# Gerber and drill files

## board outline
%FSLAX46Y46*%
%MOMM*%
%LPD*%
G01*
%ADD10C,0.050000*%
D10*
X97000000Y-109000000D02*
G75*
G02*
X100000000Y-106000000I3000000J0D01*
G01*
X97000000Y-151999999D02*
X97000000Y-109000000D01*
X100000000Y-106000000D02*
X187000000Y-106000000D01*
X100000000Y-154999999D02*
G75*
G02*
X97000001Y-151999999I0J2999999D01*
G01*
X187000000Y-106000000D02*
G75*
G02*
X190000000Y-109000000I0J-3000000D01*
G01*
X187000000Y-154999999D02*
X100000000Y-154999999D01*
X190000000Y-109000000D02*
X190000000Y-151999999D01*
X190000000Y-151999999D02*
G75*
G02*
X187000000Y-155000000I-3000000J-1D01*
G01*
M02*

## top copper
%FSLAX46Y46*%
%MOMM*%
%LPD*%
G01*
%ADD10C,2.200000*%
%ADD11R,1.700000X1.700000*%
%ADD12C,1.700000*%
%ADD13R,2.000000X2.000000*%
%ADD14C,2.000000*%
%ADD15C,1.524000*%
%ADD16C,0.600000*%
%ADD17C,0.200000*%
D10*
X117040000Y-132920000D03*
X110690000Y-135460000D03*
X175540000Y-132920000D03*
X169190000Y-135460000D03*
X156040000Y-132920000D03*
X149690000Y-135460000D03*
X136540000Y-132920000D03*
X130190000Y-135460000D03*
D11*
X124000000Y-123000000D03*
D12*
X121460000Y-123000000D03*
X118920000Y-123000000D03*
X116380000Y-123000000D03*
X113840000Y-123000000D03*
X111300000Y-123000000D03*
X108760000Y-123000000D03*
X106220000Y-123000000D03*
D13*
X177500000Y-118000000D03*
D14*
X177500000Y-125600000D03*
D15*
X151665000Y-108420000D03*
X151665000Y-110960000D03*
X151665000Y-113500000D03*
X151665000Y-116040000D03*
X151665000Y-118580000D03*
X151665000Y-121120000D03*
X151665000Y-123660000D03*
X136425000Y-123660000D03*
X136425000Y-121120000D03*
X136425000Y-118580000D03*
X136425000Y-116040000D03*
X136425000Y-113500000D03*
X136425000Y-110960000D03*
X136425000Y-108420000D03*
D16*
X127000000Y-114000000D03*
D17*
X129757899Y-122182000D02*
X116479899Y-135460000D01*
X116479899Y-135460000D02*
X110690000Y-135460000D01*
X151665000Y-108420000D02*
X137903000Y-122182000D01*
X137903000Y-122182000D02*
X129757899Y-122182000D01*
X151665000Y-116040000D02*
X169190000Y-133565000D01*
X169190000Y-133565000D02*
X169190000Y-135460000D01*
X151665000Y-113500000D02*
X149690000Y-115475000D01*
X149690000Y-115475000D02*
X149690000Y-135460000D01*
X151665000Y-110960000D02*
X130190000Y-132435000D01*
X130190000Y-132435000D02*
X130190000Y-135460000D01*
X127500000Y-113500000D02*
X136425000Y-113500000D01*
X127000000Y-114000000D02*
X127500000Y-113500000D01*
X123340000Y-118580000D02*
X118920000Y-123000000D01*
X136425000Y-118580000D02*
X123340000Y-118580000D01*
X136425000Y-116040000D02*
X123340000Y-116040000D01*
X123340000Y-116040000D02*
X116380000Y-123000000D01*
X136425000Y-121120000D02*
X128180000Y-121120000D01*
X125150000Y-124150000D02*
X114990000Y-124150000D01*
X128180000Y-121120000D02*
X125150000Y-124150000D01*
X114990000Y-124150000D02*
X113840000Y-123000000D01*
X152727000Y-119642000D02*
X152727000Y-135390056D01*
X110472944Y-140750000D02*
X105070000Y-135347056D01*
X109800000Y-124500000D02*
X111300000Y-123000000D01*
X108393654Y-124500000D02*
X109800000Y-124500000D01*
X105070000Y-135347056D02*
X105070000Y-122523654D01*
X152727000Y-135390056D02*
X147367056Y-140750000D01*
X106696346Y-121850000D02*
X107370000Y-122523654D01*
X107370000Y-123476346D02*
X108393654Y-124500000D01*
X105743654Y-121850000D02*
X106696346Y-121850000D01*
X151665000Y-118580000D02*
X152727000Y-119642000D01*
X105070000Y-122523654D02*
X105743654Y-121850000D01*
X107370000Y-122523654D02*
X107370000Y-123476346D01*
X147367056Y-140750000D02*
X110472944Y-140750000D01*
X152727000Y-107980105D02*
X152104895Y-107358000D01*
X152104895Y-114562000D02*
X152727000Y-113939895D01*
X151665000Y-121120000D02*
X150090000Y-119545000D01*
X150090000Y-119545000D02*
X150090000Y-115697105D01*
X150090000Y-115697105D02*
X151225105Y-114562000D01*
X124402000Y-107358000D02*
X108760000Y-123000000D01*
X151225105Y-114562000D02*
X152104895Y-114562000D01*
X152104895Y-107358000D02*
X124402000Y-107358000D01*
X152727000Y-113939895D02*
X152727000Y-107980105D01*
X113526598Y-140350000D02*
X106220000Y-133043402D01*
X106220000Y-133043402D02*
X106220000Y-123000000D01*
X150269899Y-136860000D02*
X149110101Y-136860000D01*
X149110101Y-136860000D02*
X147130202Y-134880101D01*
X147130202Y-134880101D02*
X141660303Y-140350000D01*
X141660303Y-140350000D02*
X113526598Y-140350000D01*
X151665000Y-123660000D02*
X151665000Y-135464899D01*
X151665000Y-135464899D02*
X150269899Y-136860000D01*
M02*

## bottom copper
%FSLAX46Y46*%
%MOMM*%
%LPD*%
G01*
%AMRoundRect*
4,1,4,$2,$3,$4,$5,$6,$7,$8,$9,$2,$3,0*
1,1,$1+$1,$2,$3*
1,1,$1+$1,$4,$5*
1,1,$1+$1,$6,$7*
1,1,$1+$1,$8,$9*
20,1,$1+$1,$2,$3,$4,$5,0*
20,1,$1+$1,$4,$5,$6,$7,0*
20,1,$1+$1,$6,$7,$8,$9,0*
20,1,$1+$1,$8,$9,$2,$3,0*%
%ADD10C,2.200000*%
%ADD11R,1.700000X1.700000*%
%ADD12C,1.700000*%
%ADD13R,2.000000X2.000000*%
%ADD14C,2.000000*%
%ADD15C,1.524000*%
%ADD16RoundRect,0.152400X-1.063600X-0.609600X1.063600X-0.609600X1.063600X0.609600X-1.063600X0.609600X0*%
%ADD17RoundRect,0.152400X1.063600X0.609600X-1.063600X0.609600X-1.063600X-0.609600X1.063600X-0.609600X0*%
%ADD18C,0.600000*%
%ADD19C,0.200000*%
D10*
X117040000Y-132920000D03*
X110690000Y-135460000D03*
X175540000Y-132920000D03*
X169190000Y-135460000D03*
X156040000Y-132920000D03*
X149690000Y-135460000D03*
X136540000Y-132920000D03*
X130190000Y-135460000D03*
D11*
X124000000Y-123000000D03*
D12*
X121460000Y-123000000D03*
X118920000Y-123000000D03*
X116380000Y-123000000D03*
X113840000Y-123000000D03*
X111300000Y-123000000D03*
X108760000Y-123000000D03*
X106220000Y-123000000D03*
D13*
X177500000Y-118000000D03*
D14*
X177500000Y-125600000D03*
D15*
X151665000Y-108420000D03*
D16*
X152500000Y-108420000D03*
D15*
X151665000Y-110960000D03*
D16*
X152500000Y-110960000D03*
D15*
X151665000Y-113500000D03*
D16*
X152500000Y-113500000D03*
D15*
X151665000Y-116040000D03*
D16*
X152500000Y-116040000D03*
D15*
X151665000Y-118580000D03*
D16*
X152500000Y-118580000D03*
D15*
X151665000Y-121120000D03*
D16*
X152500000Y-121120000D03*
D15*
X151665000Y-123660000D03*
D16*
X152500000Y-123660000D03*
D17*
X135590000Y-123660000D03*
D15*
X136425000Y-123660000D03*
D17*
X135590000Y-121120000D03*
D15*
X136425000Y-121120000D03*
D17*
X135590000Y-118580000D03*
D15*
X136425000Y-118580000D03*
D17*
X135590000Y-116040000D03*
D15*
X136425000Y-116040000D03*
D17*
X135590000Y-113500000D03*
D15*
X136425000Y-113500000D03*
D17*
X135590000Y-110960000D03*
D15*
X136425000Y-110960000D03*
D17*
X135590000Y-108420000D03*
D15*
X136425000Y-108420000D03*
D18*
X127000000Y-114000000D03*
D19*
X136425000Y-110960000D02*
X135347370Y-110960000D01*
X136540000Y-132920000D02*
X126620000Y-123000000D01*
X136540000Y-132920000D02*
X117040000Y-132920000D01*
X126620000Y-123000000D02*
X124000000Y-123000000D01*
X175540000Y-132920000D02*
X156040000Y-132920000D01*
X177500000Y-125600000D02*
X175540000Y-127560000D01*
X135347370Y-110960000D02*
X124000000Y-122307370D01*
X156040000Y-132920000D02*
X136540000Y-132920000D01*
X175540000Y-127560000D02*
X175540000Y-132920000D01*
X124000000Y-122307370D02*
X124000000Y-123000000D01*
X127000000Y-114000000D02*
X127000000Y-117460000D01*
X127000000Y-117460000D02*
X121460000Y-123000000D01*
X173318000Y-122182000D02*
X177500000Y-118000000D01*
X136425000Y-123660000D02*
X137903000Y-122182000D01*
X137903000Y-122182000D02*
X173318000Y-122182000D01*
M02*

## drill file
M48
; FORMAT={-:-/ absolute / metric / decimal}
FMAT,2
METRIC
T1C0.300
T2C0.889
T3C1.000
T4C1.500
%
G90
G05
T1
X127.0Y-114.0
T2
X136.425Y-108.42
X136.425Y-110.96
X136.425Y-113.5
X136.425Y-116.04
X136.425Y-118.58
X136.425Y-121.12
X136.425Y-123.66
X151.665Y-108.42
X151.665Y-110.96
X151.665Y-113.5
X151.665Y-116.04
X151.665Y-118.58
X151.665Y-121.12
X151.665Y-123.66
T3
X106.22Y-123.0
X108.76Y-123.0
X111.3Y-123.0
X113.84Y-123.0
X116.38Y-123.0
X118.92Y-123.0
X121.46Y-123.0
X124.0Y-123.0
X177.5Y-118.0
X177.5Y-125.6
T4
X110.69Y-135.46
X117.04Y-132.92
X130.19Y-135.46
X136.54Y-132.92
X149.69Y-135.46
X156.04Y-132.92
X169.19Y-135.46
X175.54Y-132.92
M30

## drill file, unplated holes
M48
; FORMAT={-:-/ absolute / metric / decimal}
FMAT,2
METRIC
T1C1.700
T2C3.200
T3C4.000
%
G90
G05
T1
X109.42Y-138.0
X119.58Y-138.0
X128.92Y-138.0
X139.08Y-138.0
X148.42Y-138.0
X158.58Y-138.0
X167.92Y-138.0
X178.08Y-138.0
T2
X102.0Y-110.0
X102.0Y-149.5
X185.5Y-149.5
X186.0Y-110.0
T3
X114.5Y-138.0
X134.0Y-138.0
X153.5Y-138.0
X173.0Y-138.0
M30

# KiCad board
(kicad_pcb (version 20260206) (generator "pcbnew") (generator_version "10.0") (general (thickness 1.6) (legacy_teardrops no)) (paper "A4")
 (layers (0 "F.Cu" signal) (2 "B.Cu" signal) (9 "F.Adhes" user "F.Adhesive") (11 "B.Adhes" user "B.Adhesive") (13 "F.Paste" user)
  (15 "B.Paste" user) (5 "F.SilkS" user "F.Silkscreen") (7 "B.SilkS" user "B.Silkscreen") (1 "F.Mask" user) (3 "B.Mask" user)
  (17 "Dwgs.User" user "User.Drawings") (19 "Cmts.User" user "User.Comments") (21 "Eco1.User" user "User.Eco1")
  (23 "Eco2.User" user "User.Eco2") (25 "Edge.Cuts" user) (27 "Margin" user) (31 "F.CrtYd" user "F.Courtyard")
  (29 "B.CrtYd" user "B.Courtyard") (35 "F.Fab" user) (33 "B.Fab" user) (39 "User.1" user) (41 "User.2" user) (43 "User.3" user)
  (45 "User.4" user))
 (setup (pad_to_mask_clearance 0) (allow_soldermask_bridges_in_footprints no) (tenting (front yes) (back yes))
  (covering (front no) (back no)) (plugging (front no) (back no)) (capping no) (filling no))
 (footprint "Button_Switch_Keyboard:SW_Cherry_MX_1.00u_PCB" (layer "F.Cu") (at 117.04 132.92)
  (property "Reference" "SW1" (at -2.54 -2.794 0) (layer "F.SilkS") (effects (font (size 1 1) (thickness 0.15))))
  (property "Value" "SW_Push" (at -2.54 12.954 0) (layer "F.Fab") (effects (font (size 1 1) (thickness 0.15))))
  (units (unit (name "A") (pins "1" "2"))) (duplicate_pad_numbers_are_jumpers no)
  (pad "" np_thru_hole circle (at -7.62 5.08) (size 1.7 1.7) (drill 1.7) (layers "*.Cu" "*.Mask"))
  (pad "" np_thru_hole circle (at -2.54 5.08) (size 4 4) (drill 4) (layers "*.Cu" "*.Mask"))
  (pad "" np_thru_hole circle (at 2.54 5.08) (size 1.7 1.7) (drill 1.7) (layers "*.Cu" "*.Mask"))
  (pad "1" thru_hole circle (at 0 0) (size 2.2 2.2) (drill 1.5) (layers "*.Cu" "*.Mask") (remove_unused_layers no) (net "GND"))
  (pad "2" thru_hole circle (at -6.35 2.54) (size 2.2 2.2) (drill 1.5) (layers "*.Cu" "*.Mask") (remove_unused_layers no)
   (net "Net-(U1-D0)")))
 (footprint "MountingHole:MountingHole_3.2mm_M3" (layer "F.Cu") (at 186 110)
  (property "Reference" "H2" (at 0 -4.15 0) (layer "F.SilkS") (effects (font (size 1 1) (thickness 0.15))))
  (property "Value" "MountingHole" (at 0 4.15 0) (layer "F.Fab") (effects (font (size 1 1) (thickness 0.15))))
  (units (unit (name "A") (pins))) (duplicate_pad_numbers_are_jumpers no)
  (pad "" np_thru_hole circle (at 0 0) (size 3.2 3.2) (drill 3.2) (layers "*.Cu" "*.Mask")))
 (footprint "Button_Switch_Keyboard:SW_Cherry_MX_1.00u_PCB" (layer "F.Cu") (at 175.54 132.92)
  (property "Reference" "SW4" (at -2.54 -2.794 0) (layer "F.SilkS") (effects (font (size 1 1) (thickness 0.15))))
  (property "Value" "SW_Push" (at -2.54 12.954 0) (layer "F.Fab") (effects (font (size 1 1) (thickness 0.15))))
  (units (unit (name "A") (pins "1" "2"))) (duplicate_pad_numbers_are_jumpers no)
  (pad "" np_thru_hole circle (at -7.62 5.08) (size 1.7 1.7) (drill 1.7) (layers "*.Cu" "*.Mask"))
  (pad "" np_thru_hole circle (at -2.54 5.08) (size 4 4) (drill 4) (layers "*.Cu" "*.Mask"))
  (pad "" np_thru_hole circle (at 2.54 5.08) (size 1.7 1.7) (drill 1.7) (layers "*.Cu" "*.Mask"))
  (pad "1" thru_hole circle (at 0 0) (size 2.2 2.2) (drill 1.5) (layers "*.Cu" "*.Mask") (remove_unused_layers no) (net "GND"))
  (pad "2" thru_hole circle (at -6.35 2.54) (size 2.2 2.2) (drill 1.5) (layers "*.Cu" "*.Mask") (remove_unused_layers no)
   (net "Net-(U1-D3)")))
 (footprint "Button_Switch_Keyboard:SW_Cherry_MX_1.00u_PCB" (layer "F.Cu") (at 156.04 132.92)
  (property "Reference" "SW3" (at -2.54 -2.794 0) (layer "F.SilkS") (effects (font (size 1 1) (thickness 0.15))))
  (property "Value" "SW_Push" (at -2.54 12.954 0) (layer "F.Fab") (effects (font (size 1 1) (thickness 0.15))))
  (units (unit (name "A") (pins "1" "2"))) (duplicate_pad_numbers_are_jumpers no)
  (pad "" np_thru_hole circle (at -7.62 5.08) (size 1.7 1.7) (drill 1.7) (layers "*.Cu" "*.Mask"))
  (pad "" np_thru_hole circle (at -2.54 5.08) (size 4 4) (drill 4) (layers "*.Cu" "*.Mask"))
  (pad "" np_thru_hole circle (at 2.54 5.08) (size 1.7 1.7) (drill 1.7) (layers "*.Cu" "*.Mask"))
  (pad "1" thru_hole circle (at 0 0) (size 2.2 2.2) (drill 1.5) (layers "*.Cu" "*.Mask") (remove_unused_layers no) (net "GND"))
  (pad "2" thru_hole circle (at -6.35 2.54) (size 2.2 2.2) (drill 1.5) (layers "*.Cu" "*.Mask") (remove_unused_layers no)
   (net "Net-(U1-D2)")))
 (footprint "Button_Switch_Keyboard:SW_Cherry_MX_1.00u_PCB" (layer "F.Cu") (at 136.54 132.92)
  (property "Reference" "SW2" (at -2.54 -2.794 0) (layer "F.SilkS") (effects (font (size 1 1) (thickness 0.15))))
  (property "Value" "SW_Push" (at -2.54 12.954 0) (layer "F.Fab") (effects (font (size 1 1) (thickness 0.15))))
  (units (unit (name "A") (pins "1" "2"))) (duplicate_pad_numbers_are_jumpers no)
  (pad "" np_thru_hole circle (at -7.62 5.08) (size 1.7 1.7) (drill 1.7) (layers "*.Cu" "*.Mask"))
  (pad "" np_thru_hole circle (at -2.54 5.08) (size 4 4) (drill 4) (layers "*.Cu" "*.Mask"))
  (pad "" np_thru_hole circle (at 2.54 5.08) (size 1.7 1.7) (drill 1.7) (layers "*.Cu" "*.Mask"))
  (pad "1" thru_hole circle (at 0 0) (size 2.2 2.2) (drill 1.5) (layers "*.Cu" "*.Mask") (remove_unused_layers no) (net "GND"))
  (pad "2" thru_hole circle (at -6.35 2.54) (size 2.2 2.2) (drill 1.5) (layers "*.Cu" "*.Mask") (remove_unused_layers no)
   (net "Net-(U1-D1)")))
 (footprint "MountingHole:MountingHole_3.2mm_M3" (layer "F.Cu") (at 102 110)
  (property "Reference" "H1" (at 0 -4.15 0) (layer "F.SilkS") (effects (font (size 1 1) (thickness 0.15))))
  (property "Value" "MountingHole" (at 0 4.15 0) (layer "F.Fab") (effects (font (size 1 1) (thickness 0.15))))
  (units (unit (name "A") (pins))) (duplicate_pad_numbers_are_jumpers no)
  (pad "" np_thru_hole circle (at 0 0) (size 3.2 3.2) (drill 3.2) (layers "*.Cu" "*.Mask")))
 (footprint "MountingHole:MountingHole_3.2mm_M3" (layer "F.Cu") (at 185.5 149.5)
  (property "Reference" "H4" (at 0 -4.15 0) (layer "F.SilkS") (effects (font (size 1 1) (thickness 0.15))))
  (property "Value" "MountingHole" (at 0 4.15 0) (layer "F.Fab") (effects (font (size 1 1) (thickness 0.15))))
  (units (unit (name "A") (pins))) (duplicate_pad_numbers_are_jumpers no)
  (pad "" np_thru_hole circle (at 0 0) (size 3.2 3.2) (drill 3.2) (layers "*.Cu" "*.Mask")))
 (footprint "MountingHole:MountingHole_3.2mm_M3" (layer "F.Cu") (at 102 149.5)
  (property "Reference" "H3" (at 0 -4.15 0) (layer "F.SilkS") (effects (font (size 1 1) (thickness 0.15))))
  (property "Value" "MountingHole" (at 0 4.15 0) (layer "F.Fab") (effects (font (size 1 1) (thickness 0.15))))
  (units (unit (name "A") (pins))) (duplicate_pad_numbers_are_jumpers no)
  (pad "" np_thru_hole circle (at 0 0) (size 3.2 3.2) (drill 3.2) (layers "*.Cu" "*.Mask")))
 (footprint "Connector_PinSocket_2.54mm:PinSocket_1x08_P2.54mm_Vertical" (layer "B.Cu") (at 124 123 90)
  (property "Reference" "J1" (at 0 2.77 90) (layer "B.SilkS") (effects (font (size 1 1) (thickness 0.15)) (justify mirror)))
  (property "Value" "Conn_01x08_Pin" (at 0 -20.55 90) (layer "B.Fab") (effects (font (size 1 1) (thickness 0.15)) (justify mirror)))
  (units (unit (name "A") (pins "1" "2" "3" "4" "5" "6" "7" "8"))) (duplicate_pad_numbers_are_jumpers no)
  (pad "1" thru_hole rect (at 0 0 90) (size 1.7 1.7) (drill 1) (layers "*.Cu" "*.Mask") (remove_unused_layers no) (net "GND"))
  (pad "2" thru_hole circle (at 0 -2.54 90) (size 1.7 1.7) (drill 1) (layers "*.Cu" "*.Mask") (remove_unused_layers no) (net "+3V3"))
  (pad "3" thru_hole circle (at 0 -5.08 90) (size 1.7 1.7) (drill 1) (layers "*.Cu" "*.Mask") (remove_unused_layers no) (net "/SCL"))
  (pad "4" thru_hole circle (at 0 -7.62 90) (size 1.7 1.7) (drill 1) (layers "*.Cu" "*.Mask") (remove_unused_layers no) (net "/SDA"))
  (pad "5" thru_hole circle (at 0 -10.16 90) (size 1.7 1.7) (drill 1) (layers "*.Cu" "*.Mask") (remove_unused_layers no) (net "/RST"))
  (pad "6" thru_hole circle (at 0 -12.7 90) (size 1.7 1.7) (drill 1) (layers "*.Cu" "*.Mask") (remove_unused_layers no) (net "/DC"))
  (pad "7" thru_hole circle (at 0 -15.24 90) (size 1.7 1.7) (drill 1) (layers "*.Cu" "*.Mask") (remove_unused_layers no) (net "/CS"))
  (pad "8" thru_hole circle (at 0 -17.78 90) (size 1.7 1.7) (drill 1) (layers "*.Cu" "*.Mask") (remove_unused_layers no) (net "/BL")))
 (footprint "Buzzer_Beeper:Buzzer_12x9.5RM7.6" (layer "B.Cu") (at 177.5 118 -90)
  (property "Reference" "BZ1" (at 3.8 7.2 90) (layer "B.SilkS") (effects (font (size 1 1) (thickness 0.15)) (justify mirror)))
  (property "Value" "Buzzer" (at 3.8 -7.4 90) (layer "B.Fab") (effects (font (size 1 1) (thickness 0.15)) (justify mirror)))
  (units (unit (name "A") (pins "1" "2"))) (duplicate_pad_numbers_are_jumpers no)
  (pad "1" thru_hole rect (at 0 0 270) (size 2 2) (drill 1) (layers "*.Cu" "*.Mask") (remove_unused_layers no) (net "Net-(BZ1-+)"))
  (pad "2" thru_hole circle (at 7.6 0 270) (size 2 2) (drill 1) (layers "*.Cu" "*.Mask") (remove_unused_layers no) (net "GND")))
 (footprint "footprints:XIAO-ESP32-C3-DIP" (layer "B.Cu") (at 144.045 116.04 90)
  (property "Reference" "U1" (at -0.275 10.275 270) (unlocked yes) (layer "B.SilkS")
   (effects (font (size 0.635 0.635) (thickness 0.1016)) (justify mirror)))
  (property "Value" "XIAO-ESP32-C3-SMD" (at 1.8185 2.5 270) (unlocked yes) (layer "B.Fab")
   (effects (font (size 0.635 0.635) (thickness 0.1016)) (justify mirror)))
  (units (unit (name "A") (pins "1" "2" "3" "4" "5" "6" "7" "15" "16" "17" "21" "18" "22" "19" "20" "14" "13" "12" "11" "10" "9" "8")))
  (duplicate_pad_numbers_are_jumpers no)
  (pad "1" thru_hole circle (at 7.62 7.62) (size 1.524 1.524) (drill 0.889) (layers "*.Cu" "*.Mask") (remove_unused_layers no)
   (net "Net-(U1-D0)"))
  (pad "1" smd roundrect (at 7.62 8.455) (size 2.432 1.524) (layers "B.Cu" "B.Mask") (roundrect_rratio 0.1) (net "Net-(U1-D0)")
   (thermal_bridge_angle 45))
  (pad "2" thru_hole circle (at 5.08 7.62) (size 1.524 1.524) (drill 0.889) (layers "*.Cu" "*.Mask") (remove_unused_layers no)
   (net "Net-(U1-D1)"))
  (pad "2" smd roundrect (at 5.08 8.455) (size 2.432 1.524) (layers "B.Cu" "B.Mask") (roundrect_rratio 0.1) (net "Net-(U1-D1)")
   (thermal_bridge_angle 45))
  (pad "3" thru_hole circle (at 2.54 7.62) (size 1.524 1.524) (drill 0.889) (layers "*.Cu" "*.Mask") (remove_unused_layers no)
   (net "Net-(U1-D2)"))
  (pad "3" smd roundrect (at 2.54 8.455) (size 2.432 1.524) (layers "B.Cu" "B.Mask") (roundrect_rratio 0.1) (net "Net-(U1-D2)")
   (thermal_bridge_angle 45))
  (pad "4" thru_hole circle (at 0 7.62) (size 1.524 1.524) (drill 0.889) (layers "*.Cu" "*.Mask") (remove_unused_layers no)
   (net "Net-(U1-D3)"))
  (pad "4" smd roundrect (at 0 8.455) (size 2.432 1.524) (layers "B.Cu" "B.Mask") (roundrect_rratio 0.1) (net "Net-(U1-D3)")
   (thermal_bridge_angle 45))
  (pad "5" thru_hole circle (at -2.54 7.62) (size 1.524 1.524) (drill 0.889) (layers "*.Cu" "*.Mask") (remove_unused_layers no) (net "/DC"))
  (pad "5" smd roundrect (at -2.54 8.455) (size 2.432 1.524) (layers "B.Cu" "B.Mask") (roundrect_rratio 0.1) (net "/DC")
   (thermal_bridge_angle 45))
  (pad "6" thru_hole circle (at -5.08 7.62) (size 1.524 1.524) (drill 0.889) (layers "*.Cu" "*.Mask") (remove_unused_layers no) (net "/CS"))
  (pad "6" smd roundrect (at -5.08 8.455) (size 2.432 1.524) (layers "B.Cu" "B.Mask") (roundrect_rratio 0.1) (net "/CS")
   (thermal_bridge_angle 45))
  (pad "7" thru_hole circle (at -7.62 7.62) (size 1.524 1.524) (drill 0.889) (layers "*.Cu" "*.Mask") (remove_unused_layers no) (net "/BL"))
  (pad "7" smd roundrect (at -7.62 8.455) (size 2.432 1.524) (layers "B.Cu" "B.Mask") (roundrect_rratio 0.1) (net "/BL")
   (thermal_bridge_angle 45))
  (pad "8" smd roundrect (at -7.62 -8.455 180) (size 2.432 1.524) (layers "B.Cu" "B.Mask") (roundrect_rratio 0.1) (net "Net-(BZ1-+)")
   (thermal_bridge_angle 45))
  (pad "8" thru_hole circle (at -7.62 -7.62 180) (size 1.524 1.524) (drill 0.889) (layers "*.Cu" "*.Mask") (remove_unused_layers no)
   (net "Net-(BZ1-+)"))
  (pad "9" smd roundrect (at -5.08 -8.455 180) (size 2.432 1.524) (layers "B.Cu" "B.Mask") (roundrect_rratio 0.1) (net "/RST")
   (thermal_bridge_angle 45))
  (pad "9" thru_hole circle (at -5.08 -7.62 180) (size 1.524 1.524) (drill 0.889) (layers "*.Cu" "*.Mask") (remove_unused_layers no)
   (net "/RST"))
  (pad "10" smd roundrect (at -2.54 -8.455 180) (size 2.432 1.524) (layers "B.Cu" "B.Mask") (roundrect_rratio 0.1) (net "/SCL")
   (thermal_bridge_angle 45))
  (pad "10" thru_hole circle (at -2.54 -7.62 180) (size 1.524 1.524) (drill 0.889) (layers "*.Cu" "*.Mask") (remove_unused_layers no)
   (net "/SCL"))
  (pad "11" smd roundrect (at 0 -8.455 180) (size 2.432 1.524) (layers "B.Cu" "B.Mask") (roundrect_rratio 0.1) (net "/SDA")
   (thermal_bridge_angle 45))
  (pad "11" thru_hole circle (at 0 -7.62 180) (size 1.524 1.524) (drill 0.889) (layers "*.Cu" "*.Mask") (remove_unused_layers no)
   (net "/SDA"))
  (pad "12" smd roundrect (at 2.54 -8.455 180) (size 2.432 1.524) (layers "B.Cu" "B.Mask") (roundrect_rratio 0.1) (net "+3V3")
   (thermal_bridge_angle 45))
  (pad "12" thru_hole circle (at 2.54 -7.62 180) (size 1.524 1.524) (drill 0.889) (layers "*.Cu" "*.Mask") (remove_unused_layers no)
   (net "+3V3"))
  (pad "13" smd roundrect (at 5.08 -8.455 180) (size 2.432 1.524) (layers "B.Cu" "B.Mask") (roundrect_rratio 0.1) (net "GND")
   (thermal_bridge_angle 45))
  (pad "13" thru_hole circle (at 5.08 -7.62 180) (size 1.524 1.524) (drill 0.889) (layers "*.Cu" "*.Mask") (remove_unused_layers no)
   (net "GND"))
  (pad "14" smd roundrect (at 7.62 -8.455 180) (size 2.432 1.524) (layers "B.Cu" "B.Mask") (roundrect_rratio 0.1)
   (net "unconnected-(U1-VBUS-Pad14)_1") (thermal_bridge_angle 45))
  (pad "14" thru_hole circle (at 7.62 -7.62 180) (size 1.524 1.524) (drill 0.889) (layers "*.Cu" "*.Mask") (remove_unused_layers no)
   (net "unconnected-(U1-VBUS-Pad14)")))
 (gr_arc (start 97 109) (mid 97.87868 106.87868) (end 100 106) (stroke (width 0.05) (type default)) (layer "Edge.Cuts"))
 (gr_line (start 97 151.999999) (end 97 109) (stroke (width 0.05) (type default)) (layer "Edge.Cuts"))
 (gr_line (start 100 106) (end 187 106) (stroke (width 0.05) (type default)) (layer "Edge.Cuts"))
 (gr_arc (start 100 154.999999) (mid 97.87868 154.121319) (end 97 151.999999) (stroke (width 0.05) (type default)) (layer "Edge.Cuts"))
 (gr_arc (start 187 106) (mid 189.12132 106.87868) (end 190 109) (stroke (width 0.05) (type default)) (layer "Edge.Cuts"))
 (gr_line (start 187 154.999999) (end 100 154.999999) (stroke (width 0.05) (type default)) (layer "Edge.Cuts"))
 (gr_line (start 190 109) (end 190 151.999999) (stroke (width 0.05) (type default)) (layer "Edge.Cuts"))
 (gr_arc (start 190 151.999999) (mid 189.12132 154.121319) (end 187 154.999999) (stroke (width 0.05) (type default)) (layer "Edge.Cuts"))
 (segment (start 136.425 110.96) (end 135.34737 110.96) (width 0.2) (layer "B.Cu") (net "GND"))
 (segment (start 136.54 132.92) (end 126.62 123) (width 0.2) (layer "B.Cu") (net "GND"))
 (segment (start 136.54 132.92) (end 117.04 132.92) (width 0.2) (layer "B.Cu") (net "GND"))
 (segment (start 126.62 123) (end 124 123) (width 0.2) (layer "B.Cu") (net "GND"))
 (segment (start 175.54 132.92) (end 156.04 132.92) (width 0.2) (layer "B.Cu") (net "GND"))
 (segment (start 177.5 125.6) (end 175.54 127.56) (width 0.2) (layer "B.Cu") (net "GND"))
 (segment (start 135.34737 110.96) (end 124 122.30737) (width 0.2) (layer "B.Cu") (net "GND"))
 (segment (start 156.04 132.92) (end 136.54 132.92) (width 0.2) (layer "B.Cu") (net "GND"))
 (segment (start 175.54 127.56) (end 175.54 132.92) (width 0.2) (layer "B.Cu") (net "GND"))
 (segment (start 124 122.30737) (end 124 123) (width 0.2) (layer "B.Cu") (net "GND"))
 (segment (start 129.757899 122.182) (end 116.479899 135.46) (width 0.2) (layer "F.Cu") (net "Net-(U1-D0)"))
 (segment (start 116.479899 135.46) (end 110.69 135.46) (width 0.2) (layer "F.Cu") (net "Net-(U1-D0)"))
 (segment (start 151.665 108.42) (end 137.903 122.182) (width 0.2) (layer "F.Cu") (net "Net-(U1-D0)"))
 (segment (start 137.903 122.182) (end 129.757899 122.182) (width 0.2) (layer "F.Cu") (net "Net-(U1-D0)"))
 (segment (start 151.665 116.04) (end 169.19 133.565) (width 0.2) (layer "F.Cu") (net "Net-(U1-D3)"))
 (segment (start 169.19 133.565) (end 169.19 135.46) (width 0.2) (layer "F.Cu") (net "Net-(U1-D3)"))
 (segment (start 151.665 113.5) (end 149.69 115.475) (width 0.2) (layer "F.Cu") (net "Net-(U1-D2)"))
 (segment (start 149.69 115.475) (end 149.69 135.46) (width 0.2) (layer "F.Cu") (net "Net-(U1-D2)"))
 (segment (start 151.665 110.96) (end 130.19 132.435) (width 0.2) (layer "F.Cu") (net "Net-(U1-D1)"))
 (segment (start 130.19 132.435) (end 130.19 135.46) (width 0.2) (layer "F.Cu") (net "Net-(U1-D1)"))
 (segment (start 127.5 113.5) (end 136.425 113.5) (width 0.2) (layer "F.Cu") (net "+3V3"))
 (segment (start 127 114) (end 127.5 113.5) (width 0.2) (layer "F.Cu") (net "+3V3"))
 (via (at 127 114) (size 0.6) (drill 0.3) (layers "F.Cu" "B.Cu") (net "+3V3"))
 (segment (start 127 114) (end 127 117.46) (width 0.2) (layer "B.Cu") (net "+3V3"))
 (segment (start 127 117.46) (end 121.46 123) (width 0.2) (layer "B.Cu") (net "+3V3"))
 (segment (start 123.34 118.58) (end 118.92 123) (width 0.2) (layer "F.Cu") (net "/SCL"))
 (segment (start 136.425 118.58) (end 123.34 118.58) (width 0.2) (layer "F.Cu") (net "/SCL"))
 (segment (start 136.425 116.04) (end 123.34 116.04) (width 0.2) (layer "F.Cu") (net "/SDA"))
 (segment (start 123.34 116.04) (end 116.38 123) (width 0.2) (layer "F.Cu") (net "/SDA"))
 (segment (start 136.425 121.12) (end 128.18 121.12) (width 0.2) (layer "F.Cu") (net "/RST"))
 (segment (start 125.15 124.15) (end 114.99 124.15) (width 0.2) (layer "F.Cu") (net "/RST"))
 (segment (start 128.18 121.12) (end 125.15 124.15) (width 0.2) (layer "F.Cu") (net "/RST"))
 (segment (start 114.99 124.15) (end 113.84 123) (width 0.2) (layer "F.Cu") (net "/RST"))
 (segment (start 152.727 119.642) (end 152.727 135.390056) (width 0.2) (layer "F.Cu") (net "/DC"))
 (segment (start 110.472944 140.75) (end 105.07 135.347056) (width 0.2) (layer "F.Cu") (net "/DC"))
 (segment (start 109.8 124.5) (end 111.3 123) (width 0.2) (layer "F.Cu") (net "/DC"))
 (segment (start 108.393654 124.5) (end 109.8 124.5) (width 0.2) (layer "F.Cu") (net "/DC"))
 (segment (start 105.07 135.347056) (end 105.07 122.523654) (width 0.2) (layer "F.Cu") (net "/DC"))
 (segment (start 152.727 135.390056) (end 147.367056 140.75) (width 0.2) (layer "F.Cu") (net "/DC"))
 (segment (start 106.696346 121.85) (end 107.37 122.523654) (width 0.2) (layer "F.Cu") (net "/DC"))
 (segment (start 107.37 123.476346) (end 108.393654 124.5) (width 0.2) (layer "F.Cu") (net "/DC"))
 (segment (start 105.743654 121.85) (end 106.696346 121.85) (width 0.2) (layer "F.Cu") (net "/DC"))
 (segment (start 151.665 118.58) (end 152.727 119.642) (width 0.2) (layer "F.Cu") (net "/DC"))
 (segment (start 105.07 122.523654) (end 105.743654 121.85) (width 0.2) (layer "F.Cu") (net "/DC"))
 (segment (start 107.37 122.523654) (end 107.37 123.476346) (width 0.2) (layer "F.Cu") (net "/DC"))
 (segment (start 147.367056 140.75) (end 110.472944 140.75) (width 0.2) (layer "F.Cu") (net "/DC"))
 (segment (start 152.727 107.980105) (end 152.104895 107.358) (width 0.2) (layer "F.Cu") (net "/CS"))
 (segment (start 152.104895 114.562) (end 152.727 113.939895) (width 0.2) (layer "F.Cu") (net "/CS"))
 (segment (start 151.665 121.12) (end 150.09 119.545) (width 0.2) (layer "F.Cu") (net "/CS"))
 (segment (start 150.09 119.545) (end 150.09 115.697105) (width 0.2) (layer "F.Cu") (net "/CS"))
 (segment (start 150.09 115.697105) (end 151.225105 114.562) (width 0.2) (layer "F.Cu") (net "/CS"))
 (segment (start 124.402 107.358) (end 108.76 123) (width 0.2) (layer "F.Cu") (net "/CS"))
 (segment (start 151.225105 114.562) (end 152.104895 114.562) (width 0.2) (layer "F.Cu") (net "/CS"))
 (segment (start 152.104895 107.358) (end 124.402 107.358) (width 0.2) (layer "F.Cu") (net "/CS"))
 (segment (start 152.727 113.939895) (end 152.727 107.980105) (width 0.2) (layer "F.Cu") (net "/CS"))
 (segment (start 113.526598 140.35) (end 106.22 133.043402) (width 0.2) (layer "F.Cu") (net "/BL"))
 (segment (start 106.22 133.043402) (end 106.22 123) (width 0.2) (layer "F.Cu") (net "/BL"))
 (segment (start 150.269899 136.86) (end 149.110101 136.86) (width 0.2) (layer "F.Cu") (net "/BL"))
 (segment (start 149.110101 136.86) (end 147.130202 134.880101) (width 0.2) (layer "F.Cu") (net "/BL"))
 (segment (start 147.130202 134.880101) (end 141.660303 140.35) (width 0.2) (layer "F.Cu") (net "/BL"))
 (segment (start 141.660303 140.35) (end 113.526598 140.35) (width 0.2) (layer "F.Cu") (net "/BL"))
 (segment (start 151.665 123.66) (end 151.665 135.464899) (width 0.2) (layer "F.Cu") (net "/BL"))
 (segment (start 151.665 135.464899) (end 150.269899 136.86) (width 0.2) (layer "F.Cu") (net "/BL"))
 (segment (start 173.318 122.182) (end 177.5 118) (width 0.2) (layer "B.Cu") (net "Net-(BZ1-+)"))
 (segment (start 136.425 123.66) (end 137.903 122.182) (width 0.2) (layer "B.Cu") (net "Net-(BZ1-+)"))
 (segment (start 137.903 122.182) (end 173.318 122.182) (width 0.2) (layer "B.Cu") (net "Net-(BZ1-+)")))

